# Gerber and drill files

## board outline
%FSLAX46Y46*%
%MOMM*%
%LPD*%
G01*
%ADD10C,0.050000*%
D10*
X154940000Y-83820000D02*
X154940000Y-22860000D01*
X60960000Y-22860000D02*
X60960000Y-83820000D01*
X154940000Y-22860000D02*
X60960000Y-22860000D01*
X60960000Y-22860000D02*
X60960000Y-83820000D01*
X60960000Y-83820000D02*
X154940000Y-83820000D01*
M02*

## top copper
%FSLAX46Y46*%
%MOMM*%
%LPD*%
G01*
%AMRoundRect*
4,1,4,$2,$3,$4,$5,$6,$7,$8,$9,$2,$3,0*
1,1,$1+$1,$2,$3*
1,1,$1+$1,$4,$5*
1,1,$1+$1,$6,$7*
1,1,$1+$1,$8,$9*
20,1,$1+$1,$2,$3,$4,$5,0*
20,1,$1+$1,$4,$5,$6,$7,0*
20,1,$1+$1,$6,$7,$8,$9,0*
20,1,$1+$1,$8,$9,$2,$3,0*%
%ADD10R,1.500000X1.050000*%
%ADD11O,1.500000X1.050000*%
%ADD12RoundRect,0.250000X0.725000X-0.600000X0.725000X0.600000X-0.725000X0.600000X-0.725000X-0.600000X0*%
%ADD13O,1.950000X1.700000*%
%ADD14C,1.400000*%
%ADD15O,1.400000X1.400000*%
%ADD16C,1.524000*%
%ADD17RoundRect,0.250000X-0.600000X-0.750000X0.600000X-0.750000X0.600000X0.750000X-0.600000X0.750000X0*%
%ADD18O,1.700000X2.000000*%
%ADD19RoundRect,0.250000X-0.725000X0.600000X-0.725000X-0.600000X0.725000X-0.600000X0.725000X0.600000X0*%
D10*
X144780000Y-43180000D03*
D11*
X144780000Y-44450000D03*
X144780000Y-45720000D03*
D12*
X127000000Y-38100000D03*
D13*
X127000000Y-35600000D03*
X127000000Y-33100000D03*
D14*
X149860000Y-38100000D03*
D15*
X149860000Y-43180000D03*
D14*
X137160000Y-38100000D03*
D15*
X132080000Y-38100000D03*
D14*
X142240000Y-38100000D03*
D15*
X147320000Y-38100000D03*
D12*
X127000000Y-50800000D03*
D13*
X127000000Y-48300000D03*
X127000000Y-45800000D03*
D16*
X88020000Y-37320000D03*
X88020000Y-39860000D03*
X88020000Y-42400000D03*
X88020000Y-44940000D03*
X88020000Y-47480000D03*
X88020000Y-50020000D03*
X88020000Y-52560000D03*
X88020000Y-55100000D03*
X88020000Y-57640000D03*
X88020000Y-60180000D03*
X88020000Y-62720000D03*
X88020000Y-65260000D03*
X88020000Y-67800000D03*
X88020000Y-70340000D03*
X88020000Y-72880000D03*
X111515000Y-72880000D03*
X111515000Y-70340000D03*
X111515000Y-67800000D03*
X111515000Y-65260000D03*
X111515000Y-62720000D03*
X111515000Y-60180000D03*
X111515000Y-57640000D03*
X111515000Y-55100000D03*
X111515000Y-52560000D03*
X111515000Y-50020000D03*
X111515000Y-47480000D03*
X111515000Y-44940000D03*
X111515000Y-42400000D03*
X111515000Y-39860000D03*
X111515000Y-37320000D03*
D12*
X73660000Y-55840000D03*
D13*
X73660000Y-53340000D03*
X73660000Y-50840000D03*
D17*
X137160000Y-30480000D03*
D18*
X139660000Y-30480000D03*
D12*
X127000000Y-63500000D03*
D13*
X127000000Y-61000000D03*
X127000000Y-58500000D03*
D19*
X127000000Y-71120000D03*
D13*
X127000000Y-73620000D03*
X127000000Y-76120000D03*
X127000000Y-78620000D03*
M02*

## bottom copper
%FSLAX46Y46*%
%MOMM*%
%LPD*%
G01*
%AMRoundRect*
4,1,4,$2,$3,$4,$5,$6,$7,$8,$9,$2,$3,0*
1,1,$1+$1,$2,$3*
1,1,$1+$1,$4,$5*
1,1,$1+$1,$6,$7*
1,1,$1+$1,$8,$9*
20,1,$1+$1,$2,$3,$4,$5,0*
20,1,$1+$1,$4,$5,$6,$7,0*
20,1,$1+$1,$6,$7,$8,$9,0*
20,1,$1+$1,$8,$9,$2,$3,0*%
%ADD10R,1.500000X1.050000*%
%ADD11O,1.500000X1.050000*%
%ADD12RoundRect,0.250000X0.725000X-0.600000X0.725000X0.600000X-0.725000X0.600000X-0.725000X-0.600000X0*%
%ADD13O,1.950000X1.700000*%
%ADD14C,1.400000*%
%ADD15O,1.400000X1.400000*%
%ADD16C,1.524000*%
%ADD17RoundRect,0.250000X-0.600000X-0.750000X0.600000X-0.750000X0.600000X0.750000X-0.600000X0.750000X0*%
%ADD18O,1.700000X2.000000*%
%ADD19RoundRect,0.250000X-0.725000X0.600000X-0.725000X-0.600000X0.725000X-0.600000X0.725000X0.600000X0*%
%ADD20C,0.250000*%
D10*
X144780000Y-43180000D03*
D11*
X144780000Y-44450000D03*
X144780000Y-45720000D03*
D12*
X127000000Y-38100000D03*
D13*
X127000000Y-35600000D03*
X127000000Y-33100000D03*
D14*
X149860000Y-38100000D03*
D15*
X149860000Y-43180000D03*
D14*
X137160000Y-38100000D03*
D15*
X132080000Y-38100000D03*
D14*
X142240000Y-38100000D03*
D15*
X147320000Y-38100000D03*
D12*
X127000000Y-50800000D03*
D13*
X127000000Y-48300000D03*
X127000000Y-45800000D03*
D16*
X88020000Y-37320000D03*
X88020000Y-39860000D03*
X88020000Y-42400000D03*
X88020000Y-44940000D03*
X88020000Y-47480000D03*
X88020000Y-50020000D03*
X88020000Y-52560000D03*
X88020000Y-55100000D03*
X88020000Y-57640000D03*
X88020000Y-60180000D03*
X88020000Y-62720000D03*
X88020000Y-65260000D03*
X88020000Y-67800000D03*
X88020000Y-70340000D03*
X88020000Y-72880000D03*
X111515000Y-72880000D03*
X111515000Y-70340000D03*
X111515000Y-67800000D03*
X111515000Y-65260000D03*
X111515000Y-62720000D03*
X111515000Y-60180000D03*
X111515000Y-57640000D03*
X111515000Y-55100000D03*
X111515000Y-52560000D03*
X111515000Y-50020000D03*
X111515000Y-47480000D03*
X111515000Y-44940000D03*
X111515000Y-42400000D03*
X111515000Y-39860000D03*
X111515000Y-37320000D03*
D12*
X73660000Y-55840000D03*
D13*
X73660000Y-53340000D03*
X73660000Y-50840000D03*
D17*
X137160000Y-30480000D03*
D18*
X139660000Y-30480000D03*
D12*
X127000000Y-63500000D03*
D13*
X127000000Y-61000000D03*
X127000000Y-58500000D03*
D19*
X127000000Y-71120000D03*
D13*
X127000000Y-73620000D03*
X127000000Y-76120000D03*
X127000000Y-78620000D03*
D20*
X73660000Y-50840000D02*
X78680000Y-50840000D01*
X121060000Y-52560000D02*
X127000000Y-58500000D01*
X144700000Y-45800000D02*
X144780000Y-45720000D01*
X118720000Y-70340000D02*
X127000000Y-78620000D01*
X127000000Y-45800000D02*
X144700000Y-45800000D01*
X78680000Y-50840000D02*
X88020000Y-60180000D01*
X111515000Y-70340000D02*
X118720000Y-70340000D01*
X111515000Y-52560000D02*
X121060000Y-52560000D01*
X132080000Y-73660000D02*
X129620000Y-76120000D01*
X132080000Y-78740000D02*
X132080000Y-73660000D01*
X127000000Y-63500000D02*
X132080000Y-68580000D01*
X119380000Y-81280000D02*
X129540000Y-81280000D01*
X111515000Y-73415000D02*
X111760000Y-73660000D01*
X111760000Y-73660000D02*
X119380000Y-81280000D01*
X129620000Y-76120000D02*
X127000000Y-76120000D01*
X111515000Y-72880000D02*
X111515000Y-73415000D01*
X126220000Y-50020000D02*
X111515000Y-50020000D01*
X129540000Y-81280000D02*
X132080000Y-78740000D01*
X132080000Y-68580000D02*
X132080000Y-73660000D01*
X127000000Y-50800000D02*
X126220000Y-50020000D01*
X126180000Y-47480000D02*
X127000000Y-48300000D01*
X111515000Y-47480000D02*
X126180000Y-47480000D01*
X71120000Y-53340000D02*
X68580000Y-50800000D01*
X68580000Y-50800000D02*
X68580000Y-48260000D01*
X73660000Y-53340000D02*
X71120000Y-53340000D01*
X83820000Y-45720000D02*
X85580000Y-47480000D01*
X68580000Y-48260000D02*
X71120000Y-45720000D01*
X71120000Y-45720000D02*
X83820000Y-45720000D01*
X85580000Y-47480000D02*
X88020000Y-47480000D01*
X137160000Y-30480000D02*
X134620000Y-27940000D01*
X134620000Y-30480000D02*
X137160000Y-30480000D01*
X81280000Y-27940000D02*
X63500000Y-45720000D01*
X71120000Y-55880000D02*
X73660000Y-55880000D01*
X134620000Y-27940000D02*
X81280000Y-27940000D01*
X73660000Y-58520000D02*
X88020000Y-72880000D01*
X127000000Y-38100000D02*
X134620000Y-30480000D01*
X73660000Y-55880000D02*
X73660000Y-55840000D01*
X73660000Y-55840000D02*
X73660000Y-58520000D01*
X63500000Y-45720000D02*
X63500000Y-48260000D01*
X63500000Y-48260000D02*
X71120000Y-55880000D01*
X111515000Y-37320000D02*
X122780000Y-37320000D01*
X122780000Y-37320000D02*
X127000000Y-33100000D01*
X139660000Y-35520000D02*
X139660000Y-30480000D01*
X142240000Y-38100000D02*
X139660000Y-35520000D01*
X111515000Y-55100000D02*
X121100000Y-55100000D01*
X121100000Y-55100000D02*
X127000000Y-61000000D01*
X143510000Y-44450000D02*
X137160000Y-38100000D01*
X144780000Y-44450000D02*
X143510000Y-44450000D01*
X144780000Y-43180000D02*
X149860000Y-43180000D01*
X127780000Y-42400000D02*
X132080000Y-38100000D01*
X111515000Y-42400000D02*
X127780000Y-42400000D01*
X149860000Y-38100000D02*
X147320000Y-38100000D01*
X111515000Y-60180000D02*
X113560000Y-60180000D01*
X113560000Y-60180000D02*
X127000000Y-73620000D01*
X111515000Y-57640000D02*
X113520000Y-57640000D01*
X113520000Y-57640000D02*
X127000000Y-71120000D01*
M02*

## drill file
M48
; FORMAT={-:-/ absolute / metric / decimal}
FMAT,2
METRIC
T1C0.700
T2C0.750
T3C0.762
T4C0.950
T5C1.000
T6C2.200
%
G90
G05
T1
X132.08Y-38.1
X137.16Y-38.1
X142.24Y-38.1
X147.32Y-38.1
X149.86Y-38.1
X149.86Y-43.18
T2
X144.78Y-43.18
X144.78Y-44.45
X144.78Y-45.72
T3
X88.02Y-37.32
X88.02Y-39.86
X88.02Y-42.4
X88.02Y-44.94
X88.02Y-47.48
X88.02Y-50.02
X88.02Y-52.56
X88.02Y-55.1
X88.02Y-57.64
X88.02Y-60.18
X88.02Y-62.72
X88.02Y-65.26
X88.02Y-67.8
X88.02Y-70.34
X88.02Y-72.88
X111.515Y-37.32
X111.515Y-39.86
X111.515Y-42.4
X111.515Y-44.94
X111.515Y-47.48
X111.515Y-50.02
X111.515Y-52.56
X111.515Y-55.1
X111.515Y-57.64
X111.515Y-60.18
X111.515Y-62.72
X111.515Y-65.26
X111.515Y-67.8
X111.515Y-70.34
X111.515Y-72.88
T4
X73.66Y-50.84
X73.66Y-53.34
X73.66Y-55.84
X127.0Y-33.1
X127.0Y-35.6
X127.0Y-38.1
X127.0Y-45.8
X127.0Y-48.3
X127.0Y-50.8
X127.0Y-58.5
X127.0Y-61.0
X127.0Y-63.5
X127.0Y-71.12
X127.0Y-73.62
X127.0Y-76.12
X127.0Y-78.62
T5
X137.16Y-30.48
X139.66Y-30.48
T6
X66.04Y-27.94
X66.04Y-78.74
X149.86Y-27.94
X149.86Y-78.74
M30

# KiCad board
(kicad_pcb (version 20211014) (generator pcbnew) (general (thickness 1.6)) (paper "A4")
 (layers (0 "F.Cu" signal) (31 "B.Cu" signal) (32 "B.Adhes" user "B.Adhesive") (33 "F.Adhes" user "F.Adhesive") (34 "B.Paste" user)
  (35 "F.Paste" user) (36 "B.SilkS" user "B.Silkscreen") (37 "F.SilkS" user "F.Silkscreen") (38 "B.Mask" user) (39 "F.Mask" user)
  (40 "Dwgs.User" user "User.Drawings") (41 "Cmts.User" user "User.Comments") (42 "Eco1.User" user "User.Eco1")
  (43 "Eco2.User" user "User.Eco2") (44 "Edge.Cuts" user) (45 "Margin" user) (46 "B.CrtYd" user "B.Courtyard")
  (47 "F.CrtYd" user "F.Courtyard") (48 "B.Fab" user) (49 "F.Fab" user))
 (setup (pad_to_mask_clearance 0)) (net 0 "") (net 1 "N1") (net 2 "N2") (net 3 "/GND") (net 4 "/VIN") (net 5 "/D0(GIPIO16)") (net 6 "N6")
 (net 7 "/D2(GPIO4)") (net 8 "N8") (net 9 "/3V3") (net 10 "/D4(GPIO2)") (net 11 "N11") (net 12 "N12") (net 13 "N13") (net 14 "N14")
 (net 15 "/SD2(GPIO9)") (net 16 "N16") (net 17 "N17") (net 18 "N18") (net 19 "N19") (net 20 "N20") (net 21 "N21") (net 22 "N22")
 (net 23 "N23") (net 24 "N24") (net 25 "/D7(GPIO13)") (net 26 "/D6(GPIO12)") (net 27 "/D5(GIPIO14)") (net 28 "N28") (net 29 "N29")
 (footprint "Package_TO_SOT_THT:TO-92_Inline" (layer "F.Cu") (at 144.78 43.18 -90)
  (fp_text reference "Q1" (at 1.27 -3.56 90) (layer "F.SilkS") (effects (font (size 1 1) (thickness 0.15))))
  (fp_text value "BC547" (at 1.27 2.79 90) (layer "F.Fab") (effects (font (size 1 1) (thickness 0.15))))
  (pad "1" thru_hole rect (at 0 0 270) (size 1.05 1.5) (drill 0.75) (layers *.Cu *.Mask) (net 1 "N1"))
  (pad "2" thru_hole oval (at 1.27 0 270) (size 1.05 1.5) (drill 0.75) (layers *.Cu *.Mask) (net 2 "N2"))
  (pad "3" thru_hole oval (at 2.54 0 270) (size 1.05 1.5) (drill 0.75) (layers *.Cu *.Mask) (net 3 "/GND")))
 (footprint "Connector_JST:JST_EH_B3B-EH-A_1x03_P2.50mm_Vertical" (layer "F.Cu") (at 127 38.1 90)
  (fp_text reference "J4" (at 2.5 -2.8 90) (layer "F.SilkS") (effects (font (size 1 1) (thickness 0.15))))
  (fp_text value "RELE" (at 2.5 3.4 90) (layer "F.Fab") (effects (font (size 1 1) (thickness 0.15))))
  (pad "1" thru_hole roundrect (at 0 0 90) (size 1.7 1.95) (drill 0.95) (layers *.Cu *.Mask) (roundrect_rratio 0.147059) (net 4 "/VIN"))
  (pad "2" thru_hole oval (at 2.5 0 90) (size 1.7 1.95) (drill 0.95) (layers *.Cu *.Mask) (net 3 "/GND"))
  (pad "3" thru_hole oval (at 5 0 90) (size 1.7 1.95) (drill 0.95) (layers *.Cu *.Mask) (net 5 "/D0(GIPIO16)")))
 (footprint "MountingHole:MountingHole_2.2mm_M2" (layer "F.Cu") (at 149.86 78.74)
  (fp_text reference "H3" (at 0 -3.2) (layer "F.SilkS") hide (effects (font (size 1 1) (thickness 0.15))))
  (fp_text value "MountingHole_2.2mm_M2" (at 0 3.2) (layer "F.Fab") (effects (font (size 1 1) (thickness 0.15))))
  (pad "" np_thru_hole circle (at 0 0) (size 2.2 2.2) (drill 2.2) (layers *.Cu *.Mask)))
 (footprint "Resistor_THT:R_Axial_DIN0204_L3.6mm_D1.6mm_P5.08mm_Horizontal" (layer "F.Cu") (at 149.86 38.1 -90)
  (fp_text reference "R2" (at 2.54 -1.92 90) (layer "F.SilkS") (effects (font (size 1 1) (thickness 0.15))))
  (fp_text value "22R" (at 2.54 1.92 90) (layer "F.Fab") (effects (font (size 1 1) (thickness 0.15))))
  (pad "1" thru_hole circle (at 0 0 270) (size 1.4 1.4) (drill 0.7) (layers *.Cu *.Mask) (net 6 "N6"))
  (pad "2" thru_hole oval (at 5.08 0 270) (size 1.4 1.4) (drill 0.7) (layers *.Cu *.Mask) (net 1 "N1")))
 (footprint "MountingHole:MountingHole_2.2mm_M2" (layer "F.Cu") (at 66.04 78.74)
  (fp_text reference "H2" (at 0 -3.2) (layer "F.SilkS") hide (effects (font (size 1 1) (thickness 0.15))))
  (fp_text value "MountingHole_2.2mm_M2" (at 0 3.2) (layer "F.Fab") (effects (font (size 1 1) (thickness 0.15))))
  (pad "" np_thru_hole circle (at 0 0) (size 2.2 2.2) (drill 2.2) (layers *.Cu *.Mask)))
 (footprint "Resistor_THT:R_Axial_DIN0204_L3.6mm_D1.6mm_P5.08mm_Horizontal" (layer "F.Cu") (at 137.16 38.1 180)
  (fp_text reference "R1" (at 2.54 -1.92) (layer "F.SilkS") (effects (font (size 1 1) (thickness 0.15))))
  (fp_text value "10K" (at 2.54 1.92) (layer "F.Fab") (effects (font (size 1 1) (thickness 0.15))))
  (pad "1" thru_hole circle (at 0 0 180) (size 1.4 1.4) (drill 0.7) (layers *.Cu *.Mask) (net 2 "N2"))
  (pad "2" thru_hole oval (at 5.08 0 180) (size 1.4 1.4) (drill 0.7) (layers *.Cu *.Mask) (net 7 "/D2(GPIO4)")))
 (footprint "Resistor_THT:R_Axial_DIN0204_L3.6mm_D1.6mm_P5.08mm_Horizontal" (layer "F.Cu") (at 142.24 38.1)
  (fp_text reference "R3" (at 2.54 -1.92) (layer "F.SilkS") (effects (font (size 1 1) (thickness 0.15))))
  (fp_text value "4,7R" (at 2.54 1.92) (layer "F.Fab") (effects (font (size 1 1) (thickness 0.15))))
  (pad "1" thru_hole circle (at 0 0) (size 1.4 1.4) (drill 0.7) (layers *.Cu *.Mask) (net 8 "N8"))
  (pad "2" thru_hole oval (at 5.08 0) (size 1.4 1.4) (drill 0.7) (layers *.Cu *.Mask) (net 6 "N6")))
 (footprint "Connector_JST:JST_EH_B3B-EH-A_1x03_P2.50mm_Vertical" (layer "F.Cu") (at 127 50.8 90)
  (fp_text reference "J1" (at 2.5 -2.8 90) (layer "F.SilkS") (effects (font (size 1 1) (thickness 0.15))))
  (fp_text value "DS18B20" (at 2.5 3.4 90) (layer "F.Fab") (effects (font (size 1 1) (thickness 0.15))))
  (pad "1" thru_hole roundrect (at 0 0 90) (size 1.7 1.95) (drill 0.95) (layers *.Cu *.Mask) (roundrect_rratio 0.147059) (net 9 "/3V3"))
  (pad "2" thru_hole oval (at 2.5 0 90) (size 1.7 1.95) (drill 0.95) (layers *.Cu *.Mask) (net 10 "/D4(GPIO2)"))
  (pad "3" thru_hole oval (at 5 0 90) (size 1.7 1.95) (drill 0.95) (layers *.Cu *.Mask) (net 3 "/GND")))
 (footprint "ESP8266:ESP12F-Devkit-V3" (layer "F.Cu") (at 100.085 56.37)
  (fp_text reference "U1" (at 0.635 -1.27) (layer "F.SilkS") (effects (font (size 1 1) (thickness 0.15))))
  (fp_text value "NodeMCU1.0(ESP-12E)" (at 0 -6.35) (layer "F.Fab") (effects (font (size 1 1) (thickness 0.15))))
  (pad "1" thru_hole circle locked (at -12.065 -19.05) (size 1.524 1.524) (drill 0.762) (layers *.Cu *.Mask "F.SilkS") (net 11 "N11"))
  (pad "2" thru_hole circle locked (at -12.065 -16.51) (size 1.524 1.524) (drill 0.762) (layers *.Cu *.Mask "F.SilkS") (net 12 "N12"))
  (pad "3" thru_hole circle locked (at -12.065 -13.97) (size 1.524 1.524) (drill 0.762) (layers *.Cu *.Mask "F.SilkS") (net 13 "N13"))
  (pad "4" thru_hole circle locked (at -12.065 -11.43) (size 1.524 1.524) (drill 0.762) (layers *.Cu *.Mask "F.SilkS") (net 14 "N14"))
  (pad "5" thru_hole circle locked (at -12.065 -8.89) (size 1.524 1.524) (drill 0.762) (layers *.Cu *.Mask "F.SilkS") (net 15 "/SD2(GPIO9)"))
  (pad "6" thru_hole circle locked (at -12.065 -6.35) (size 1.524 1.524) (drill 0.762) (layers *.Cu *.Mask "F.SilkS") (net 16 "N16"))
  (pad "7" thru_hole circle locked (at -12.065 -3.81) (size 1.524 1.524) (drill 0.762) (layers *.Cu *.Mask "F.SilkS") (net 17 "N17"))
  (pad "8" thru_hole circle locked (at -12.065 -1.27) (size 1.524 1.524) (drill 0.762) (layers *.Cu *.Mask "F.SilkS") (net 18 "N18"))
  (pad "9" thru_hole circle locked (at -12.065 1.27) (size 1.524 1.524) (drill 0.762) (layers *.Cu *.Mask "F.SilkS") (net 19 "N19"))
  (pad "10" thru_hole circle locked (at -12.065 3.81) (size 1.524 1.524) (drill 0.762) (layers *.Cu *.Mask "F.SilkS") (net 3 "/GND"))
  (pad "11" thru_hole circle locked (at -12.065 6.35) (size 1.524 1.524) (drill 0.762) (layers *.Cu *.Mask "F.SilkS") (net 9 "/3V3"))
  (pad "12" thru_hole circle locked (at -12.065 8.89) (size 1.524 1.524) (drill 0.762) (layers *.Cu *.Mask "F.SilkS") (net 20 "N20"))
  (pad "13" thru_hole circle locked (at -12.065 11.43) (size 1.524 1.524) (drill 0.762) (layers *.Cu *.Mask "F.SilkS") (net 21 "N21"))
  (pad "14" thru_hole circle locked (at -12.065 13.97) (size 1.524 1.524) (drill 0.762) (layers *.Cu *.Mask "F.SilkS") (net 3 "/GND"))
  (pad "15" thru_hole circle locked (at -12.065 16.51) (size 1.524 1.524) (drill 0.762) (layers *.Cu *.Mask "F.SilkS") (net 4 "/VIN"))
  (pad "16" thru_hole circle locked (at 11.43 16.51) (size 1.524 1.524) (drill 0.762) (layers *.Cu *.Mask "F.SilkS") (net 9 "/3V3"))
  (pad "17" thru_hole circle locked (at 11.43 13.97) (size 1.524 1.524) (drill 0.762) (layers *.Cu *.Mask "F.SilkS") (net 3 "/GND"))
  (pad "18" thru_hole circle locked (at 11.43 11.43) (size 1.524 1.524) (drill 0.762) (layers *.Cu *.Mask "F.SilkS") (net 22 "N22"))
  (pad "19" thru_hole circle locked (at 11.43 8.89) (size 1.524 1.524) (drill 0.762) (layers *.Cu *.Mask "F.SilkS") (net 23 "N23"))
  (pad "20" thru_hole circle locked (at 11.43 6.35) (size 1.524 1.524) (drill 0.762) (layers *.Cu *.Mask "F.SilkS") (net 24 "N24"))
  (pad "21" thru_hole circle locked (at 11.43 3.81) (size 1.524 1.524) (drill 0.762) (layers *.Cu *.Mask "F.SilkS") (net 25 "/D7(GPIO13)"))
  (pad "22" thru_hole circle locked (at 11.43 1.27) (size 1.524 1.524) (drill 0.762) (layers *.Cu *.Mask "F.SilkS") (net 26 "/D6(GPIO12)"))
  (pad "23" thru_hole circle locked (at 11.43 -1.27) (size 1.524 1.524) (drill 0.762) (layers *.Cu *.Mask "F.SilkS") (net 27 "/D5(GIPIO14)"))
  (pad "24" thru_hole circle locked (at 11.43 -3.81) (size 1.524 1.524) (drill 0.762) (layers *.Cu *.Mask "F.SilkS") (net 3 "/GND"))
  (pad "25" thru_hole circle locked (at 11.43 -6.35) (size 1.524 1.524) (drill 0.762) (layers *.Cu *.Mask "F.SilkS") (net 9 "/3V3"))
  (pad "26" thru_hole circle locked (at 11.43 -8.89) (size 1.524 1.524) (drill 0.762) (layers *.Cu *.Mask "F.SilkS") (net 10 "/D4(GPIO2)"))
  (pad "27" thru_hole circle locked (at 11.43 -11.43) (size 1.524 1.524) (drill 0.762) (layers *.Cu *.Mask "F.SilkS") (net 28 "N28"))
  (pad "28" thru_hole circle locked (at 11.43 -13.97) (size 1.524 1.524) (drill 0.762) (layers *.Cu *.Mask "F.SilkS") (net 7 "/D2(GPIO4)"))
  (pad "29" thru_hole circle locked (at 11.43 -16.51) (size 1.524 1.524) (drill 0.762) (layers *.Cu *.Mask "F.SilkS") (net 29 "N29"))
  (pad "30" thru_hole circle locked (at 11.43 -19.05) (size 1.524 1.524) (drill 0.762) (layers *.Cu *.Mask "F.SilkS") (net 5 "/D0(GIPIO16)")))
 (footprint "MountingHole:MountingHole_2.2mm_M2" (layer "F.Cu") (at 149.86 27.94)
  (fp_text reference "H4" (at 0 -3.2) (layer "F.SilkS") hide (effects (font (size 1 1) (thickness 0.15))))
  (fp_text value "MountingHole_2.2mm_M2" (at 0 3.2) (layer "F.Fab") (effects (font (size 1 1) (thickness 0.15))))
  (pad "" np_thru_hole circle (at 0 0) (size 2.2 2.2) (drill 2.2) (layers *.Cu *.Mask)))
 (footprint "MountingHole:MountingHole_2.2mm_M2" (layer "F.Cu") (at 66.04 27.94)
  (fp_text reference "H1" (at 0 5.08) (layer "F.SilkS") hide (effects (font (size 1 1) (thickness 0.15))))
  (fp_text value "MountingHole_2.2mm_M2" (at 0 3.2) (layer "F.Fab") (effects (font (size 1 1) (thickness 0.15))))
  (pad "" np_thru_hole circle (at 0 0) (size 2.2 2.2) (drill 2.2) (layers *.Cu *.Mask)))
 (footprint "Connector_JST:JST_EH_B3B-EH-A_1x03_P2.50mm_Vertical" (layer "F.Cu") (at 73.66 55.84 90)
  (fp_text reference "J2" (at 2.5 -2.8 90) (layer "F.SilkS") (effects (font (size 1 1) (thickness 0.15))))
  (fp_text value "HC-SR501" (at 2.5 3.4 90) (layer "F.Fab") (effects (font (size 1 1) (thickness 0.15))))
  (pad "1" thru_hole roundrect (at 0 0 90) (size 1.7 1.95) (drill 0.95) (layers *.Cu *.Mask) (roundrect_rratio 0.147059) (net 4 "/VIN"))
  (pad "2" thru_hole oval (at 2.5 0 90) (size 1.7 1.95) (drill 0.95) (layers *.Cu *.Mask) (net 15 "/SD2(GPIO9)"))
  (pad "3" thru_hole oval (at 5 0 90) (size 1.7 1.95) (drill 0.95) (layers *.Cu *.Mask) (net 3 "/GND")))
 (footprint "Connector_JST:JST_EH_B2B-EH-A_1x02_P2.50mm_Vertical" (layer "F.Cu") (at 137.16 30.48)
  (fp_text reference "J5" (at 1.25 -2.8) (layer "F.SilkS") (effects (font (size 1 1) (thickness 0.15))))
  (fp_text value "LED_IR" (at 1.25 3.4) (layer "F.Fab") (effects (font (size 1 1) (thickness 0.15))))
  (pad "1" thru_hole roundrect (at 0 0) (size 1.7 2) (drill 1) (layers *.Cu *.Mask) (roundrect_rratio 0.147059) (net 4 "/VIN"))
  (pad "2" thru_hole oval (at 2.5 0) (size 1.7 2) (drill 1) (layers *.Cu *.Mask) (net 8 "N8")))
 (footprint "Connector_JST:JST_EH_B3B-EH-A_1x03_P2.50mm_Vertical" (layer "F.Cu") (at 127 63.5 90)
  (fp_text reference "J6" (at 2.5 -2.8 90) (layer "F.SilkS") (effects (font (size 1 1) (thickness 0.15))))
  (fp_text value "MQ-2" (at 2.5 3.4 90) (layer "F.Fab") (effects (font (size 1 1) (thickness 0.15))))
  (pad "1" thru_hole roundrect (at 0 0 90) (size 1.7 1.95) (drill 0.95) (layers *.Cu *.Mask) (roundrect_rratio 0.147059) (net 9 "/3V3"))
  (pad "2" thru_hole oval (at 2.5 0 90) (size 1.7 1.95) (drill 0.95) (layers *.Cu *.Mask) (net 27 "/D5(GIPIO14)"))
  (pad "3" thru_hole oval (at 5 0 90) (size 1.7 1.95) (drill 0.95) (layers *.Cu *.Mask) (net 3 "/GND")))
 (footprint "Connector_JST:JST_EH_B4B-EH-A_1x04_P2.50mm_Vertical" (layer "F.Cu") (at 127 71.12 -90)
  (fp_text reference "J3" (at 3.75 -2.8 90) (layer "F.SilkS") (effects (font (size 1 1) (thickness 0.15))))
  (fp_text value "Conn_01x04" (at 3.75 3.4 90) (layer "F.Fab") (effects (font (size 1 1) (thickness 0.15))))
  (pad "1" thru_hole roundrect (at 0 0 270) (size 1.7 1.95) (drill 0.95) (layers *.Cu *.Mask) (roundrect_rratio 0.147059)
   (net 26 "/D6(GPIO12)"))
  (pad "2" thru_hole oval (at 2.5 0 270) (size 1.7 1.95) (drill 0.95) (layers *.Cu *.Mask) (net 25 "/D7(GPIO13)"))
  (pad "3" thru_hole oval (at 5 0 270) (size 1.7 1.95) (drill 0.95) (layers *.Cu *.Mask) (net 9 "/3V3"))
  (pad "4" thru_hole oval (at 7.5 0 270) (size 1.7 1.95) (drill 0.95) (layers *.Cu *.Mask) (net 3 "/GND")))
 (gr_line (start 154.94 83.82) (end 154.94 22.86) (layer "Edge.Cuts") (width 0.05))
 (gr_line (start 60.96 22.86) (end 60.96 83.82) (layer "Edge.Cuts") (width 0.05))
 (gr_line (start 154.94 22.86) (end 60.96 22.86) (layer "Edge.Cuts") (width 0.05))
 (gr_line (start 60.96 22.86) (end 60.96 83.82) (layer "Edge.Cuts") (width 0.05))
 (gr_line (start 60.96 83.82) (end 154.94 83.82) (layer "Edge.Cuts") (width 0.05))
 (segment (start 73.66 50.84) (end 78.68 50.84) (width 0.25) (layer "B.Cu") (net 3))
 (segment (start 121.06 52.56) (end 127 58.5) (width 0.25) (layer "B.Cu") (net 3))
 (segment (start 144.7 45.8) (end 144.78 45.72) (width 0.25) (layer "B.Cu") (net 3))
 (segment (start 118.72 70.34) (end 127 78.62) (width 0.25) (layer "B.Cu") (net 3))
 (segment (start 127 45.8) (end 144.7 45.8) (width 0.25) (layer "B.Cu") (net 3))
 (segment (start 78.68 50.84) (end 88.02 60.18) (width 0.25) (layer "B.Cu") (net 3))
 (segment (start 111.515 70.34) (end 118.72 70.34) (width 0.25) (layer "B.Cu") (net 3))
 (segment (start 111.515 52.56) (end 121.06 52.56) (width 0.25) (layer "B.Cu") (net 3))
 (segment (start 132.08 73.66) (end 129.62 76.12) (width 0.25) (layer "B.Cu") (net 9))
 (segment (start 132.08 78.74) (end 132.08 73.66) (width 0.25) (layer "B.Cu") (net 9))
 (segment (start 127 63.5) (end 132.08 68.58) (width 0.25) (layer "B.Cu") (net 9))
 (segment (start 119.38 81.28) (end 129.54 81.28) (width 0.25) (layer "B.Cu") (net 9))
 (segment (start 111.515 73.415) (end 111.76 73.66) (width 0.25) (layer "B.Cu") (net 9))
 (segment (start 111.76 73.66) (end 119.38 81.28) (width 0.25) (layer "B.Cu") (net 9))
 (segment (start 129.62 76.12) (end 127 76.12) (width 0.25) (layer "B.Cu") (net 9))
 (segment (start 111.515 72.88) (end 111.515 73.415) (width 0.25) (layer "B.Cu") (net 9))
 (segment (start 126.22 50.02) (end 111.515 50.02) (width 0.25) (layer "B.Cu") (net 9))
 (segment (start 129.54 81.28) (end 132.08 78.74) (width 0.25) (layer "B.Cu") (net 9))
 (segment (start 132.08 68.58) (end 132.08 73.66) (width 0.25) (layer "B.Cu") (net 9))
 (segment (start 127 50.8) (end 126.22 50.02) (width 0.25) (layer "B.Cu") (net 9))
 (segment (start 126.18 47.48) (end 127 48.3) (width 0.25) (layer "B.Cu") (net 10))
 (segment (start 111.515 47.48) (end 126.18 47.48) (width 0.25) (layer "B.Cu") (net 10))
 (segment (start 71.12 53.34) (end 68.58 50.8) (width 0.25) (layer "B.Cu") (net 15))
 (segment (start 68.58 50.8) (end 68.58 48.26) (width 0.25) (layer "B.Cu") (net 15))
 (segment (start 73.66 53.34) (end 71.12 53.34) (width 0.25) (layer "B.Cu") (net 15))
 (segment (start 83.82 45.72) (end 85.58 47.48) (width 0.25) (layer "B.Cu") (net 15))
 (segment (start 68.58 48.26) (end 71.12 45.72) (width 0.25) (layer "B.Cu") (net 15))
 (segment (start 71.12 45.72) (end 83.82 45.72) (width 0.25) (layer "B.Cu") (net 15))
 (segment (start 85.58 47.48) (end 88.02 47.48) (width 0.25) (layer "B.Cu") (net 15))
 (segment (start 137.16 30.48) (end 134.62 27.94) (width 0.25) (layer "B.Cu") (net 4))
 (segment (start 134.62 30.48) (end 137.16 30.48) (width 0.25) (layer "B.Cu") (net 4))
 (segment (start 81.28 27.94) (end 63.5 45.72) (width 0.25) (layer "B.Cu") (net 4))
 (segment (start 71.12 55.88) (end 73.66 55.88) (width 0.25) (layer "B.Cu") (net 4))
 (segment (start 134.62 27.94) (end 81.28 27.94) (width 0.25) (layer "B.Cu") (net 4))
 (segment (start 73.66 58.52) (end 88.02 72.88) (width 0.25) (layer "B.Cu") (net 4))
 (segment (start 127 38.1) (end 134.62 30.48) (width 0.25) (layer "B.Cu") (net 4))
 (segment (start 73.66 55.88) (end 73.66 55.84) (width 0.25) (layer "B.Cu") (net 4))
 (segment (start 73.66 55.84) (end 73.66 58.52) (width 0.25) (layer "B.Cu") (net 4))
 (segment (start 63.5 45.72) (end 63.5 48.26) (width 0.25) (layer "B.Cu") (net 4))
 (segment (start 63.5 48.26) (end 71.12 55.88) (width 0.25) (layer "B.Cu") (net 4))
 (segment (start 111.515 37.32) (end 122.78 37.32) (width 0.25) (layer "B.Cu") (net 5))
 (segment (start 122.78 37.32) (end 127 33.1) (width 0.25) (layer "B.Cu") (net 5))
 (segment (start 139.66 35.52) (end 139.66 30.48) (width 0.25) (layer "B.Cu") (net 8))
 (segment (start 142.24 38.1) (end 139.66 35.52) (width 0.25) (layer "B.Cu") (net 8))
 (segment (start 111.515 55.1) (end 121.1 55.1) (width 0.25) (layer "B.Cu") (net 27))
 (segment (start 121.1 55.1) (end 127 61) (width 0.25) (layer "B.Cu") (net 27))
 (segment (start 143.51 44.45) (end 137.16 38.1) (width 0.25) (layer "B.Cu") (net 2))
 (segment (start 144.78 44.45) (end 143.51 44.45) (width 0.25) (layer "B.Cu") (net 2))
 (segment (start 144.78 43.18) (end 149.86 43.18) (width 0.25) (layer "B.Cu") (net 1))
 (segment (start 127.78 42.4) (end 132.08 38.1) (width 0.25) (layer "B.Cu") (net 7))
 (segment (start 111.515 42.4) (end 127.78 42.4) (width 0.25) (layer "B.Cu") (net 7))
 (segment (start 149.86 38.1) (end 147.32 38.1) (width 0.25) (layer "B.Cu") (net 6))
 (segment (start 111.515 60.18) (end 113.56 60.18) (width 0.25) (layer "B.Cu") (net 25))
 (segment (start 113.56 60.18) (end 127 73.62) (width 0.25) (layer "B.Cu") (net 25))
 (segment (start 111.515 57.64) (end 113.52 57.64) (width 0.25) (layer "B.Cu") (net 26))
 (segment (start 113.52 57.64) (end 127 71.12) (width 0.25) (layer "B.Cu") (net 26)))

